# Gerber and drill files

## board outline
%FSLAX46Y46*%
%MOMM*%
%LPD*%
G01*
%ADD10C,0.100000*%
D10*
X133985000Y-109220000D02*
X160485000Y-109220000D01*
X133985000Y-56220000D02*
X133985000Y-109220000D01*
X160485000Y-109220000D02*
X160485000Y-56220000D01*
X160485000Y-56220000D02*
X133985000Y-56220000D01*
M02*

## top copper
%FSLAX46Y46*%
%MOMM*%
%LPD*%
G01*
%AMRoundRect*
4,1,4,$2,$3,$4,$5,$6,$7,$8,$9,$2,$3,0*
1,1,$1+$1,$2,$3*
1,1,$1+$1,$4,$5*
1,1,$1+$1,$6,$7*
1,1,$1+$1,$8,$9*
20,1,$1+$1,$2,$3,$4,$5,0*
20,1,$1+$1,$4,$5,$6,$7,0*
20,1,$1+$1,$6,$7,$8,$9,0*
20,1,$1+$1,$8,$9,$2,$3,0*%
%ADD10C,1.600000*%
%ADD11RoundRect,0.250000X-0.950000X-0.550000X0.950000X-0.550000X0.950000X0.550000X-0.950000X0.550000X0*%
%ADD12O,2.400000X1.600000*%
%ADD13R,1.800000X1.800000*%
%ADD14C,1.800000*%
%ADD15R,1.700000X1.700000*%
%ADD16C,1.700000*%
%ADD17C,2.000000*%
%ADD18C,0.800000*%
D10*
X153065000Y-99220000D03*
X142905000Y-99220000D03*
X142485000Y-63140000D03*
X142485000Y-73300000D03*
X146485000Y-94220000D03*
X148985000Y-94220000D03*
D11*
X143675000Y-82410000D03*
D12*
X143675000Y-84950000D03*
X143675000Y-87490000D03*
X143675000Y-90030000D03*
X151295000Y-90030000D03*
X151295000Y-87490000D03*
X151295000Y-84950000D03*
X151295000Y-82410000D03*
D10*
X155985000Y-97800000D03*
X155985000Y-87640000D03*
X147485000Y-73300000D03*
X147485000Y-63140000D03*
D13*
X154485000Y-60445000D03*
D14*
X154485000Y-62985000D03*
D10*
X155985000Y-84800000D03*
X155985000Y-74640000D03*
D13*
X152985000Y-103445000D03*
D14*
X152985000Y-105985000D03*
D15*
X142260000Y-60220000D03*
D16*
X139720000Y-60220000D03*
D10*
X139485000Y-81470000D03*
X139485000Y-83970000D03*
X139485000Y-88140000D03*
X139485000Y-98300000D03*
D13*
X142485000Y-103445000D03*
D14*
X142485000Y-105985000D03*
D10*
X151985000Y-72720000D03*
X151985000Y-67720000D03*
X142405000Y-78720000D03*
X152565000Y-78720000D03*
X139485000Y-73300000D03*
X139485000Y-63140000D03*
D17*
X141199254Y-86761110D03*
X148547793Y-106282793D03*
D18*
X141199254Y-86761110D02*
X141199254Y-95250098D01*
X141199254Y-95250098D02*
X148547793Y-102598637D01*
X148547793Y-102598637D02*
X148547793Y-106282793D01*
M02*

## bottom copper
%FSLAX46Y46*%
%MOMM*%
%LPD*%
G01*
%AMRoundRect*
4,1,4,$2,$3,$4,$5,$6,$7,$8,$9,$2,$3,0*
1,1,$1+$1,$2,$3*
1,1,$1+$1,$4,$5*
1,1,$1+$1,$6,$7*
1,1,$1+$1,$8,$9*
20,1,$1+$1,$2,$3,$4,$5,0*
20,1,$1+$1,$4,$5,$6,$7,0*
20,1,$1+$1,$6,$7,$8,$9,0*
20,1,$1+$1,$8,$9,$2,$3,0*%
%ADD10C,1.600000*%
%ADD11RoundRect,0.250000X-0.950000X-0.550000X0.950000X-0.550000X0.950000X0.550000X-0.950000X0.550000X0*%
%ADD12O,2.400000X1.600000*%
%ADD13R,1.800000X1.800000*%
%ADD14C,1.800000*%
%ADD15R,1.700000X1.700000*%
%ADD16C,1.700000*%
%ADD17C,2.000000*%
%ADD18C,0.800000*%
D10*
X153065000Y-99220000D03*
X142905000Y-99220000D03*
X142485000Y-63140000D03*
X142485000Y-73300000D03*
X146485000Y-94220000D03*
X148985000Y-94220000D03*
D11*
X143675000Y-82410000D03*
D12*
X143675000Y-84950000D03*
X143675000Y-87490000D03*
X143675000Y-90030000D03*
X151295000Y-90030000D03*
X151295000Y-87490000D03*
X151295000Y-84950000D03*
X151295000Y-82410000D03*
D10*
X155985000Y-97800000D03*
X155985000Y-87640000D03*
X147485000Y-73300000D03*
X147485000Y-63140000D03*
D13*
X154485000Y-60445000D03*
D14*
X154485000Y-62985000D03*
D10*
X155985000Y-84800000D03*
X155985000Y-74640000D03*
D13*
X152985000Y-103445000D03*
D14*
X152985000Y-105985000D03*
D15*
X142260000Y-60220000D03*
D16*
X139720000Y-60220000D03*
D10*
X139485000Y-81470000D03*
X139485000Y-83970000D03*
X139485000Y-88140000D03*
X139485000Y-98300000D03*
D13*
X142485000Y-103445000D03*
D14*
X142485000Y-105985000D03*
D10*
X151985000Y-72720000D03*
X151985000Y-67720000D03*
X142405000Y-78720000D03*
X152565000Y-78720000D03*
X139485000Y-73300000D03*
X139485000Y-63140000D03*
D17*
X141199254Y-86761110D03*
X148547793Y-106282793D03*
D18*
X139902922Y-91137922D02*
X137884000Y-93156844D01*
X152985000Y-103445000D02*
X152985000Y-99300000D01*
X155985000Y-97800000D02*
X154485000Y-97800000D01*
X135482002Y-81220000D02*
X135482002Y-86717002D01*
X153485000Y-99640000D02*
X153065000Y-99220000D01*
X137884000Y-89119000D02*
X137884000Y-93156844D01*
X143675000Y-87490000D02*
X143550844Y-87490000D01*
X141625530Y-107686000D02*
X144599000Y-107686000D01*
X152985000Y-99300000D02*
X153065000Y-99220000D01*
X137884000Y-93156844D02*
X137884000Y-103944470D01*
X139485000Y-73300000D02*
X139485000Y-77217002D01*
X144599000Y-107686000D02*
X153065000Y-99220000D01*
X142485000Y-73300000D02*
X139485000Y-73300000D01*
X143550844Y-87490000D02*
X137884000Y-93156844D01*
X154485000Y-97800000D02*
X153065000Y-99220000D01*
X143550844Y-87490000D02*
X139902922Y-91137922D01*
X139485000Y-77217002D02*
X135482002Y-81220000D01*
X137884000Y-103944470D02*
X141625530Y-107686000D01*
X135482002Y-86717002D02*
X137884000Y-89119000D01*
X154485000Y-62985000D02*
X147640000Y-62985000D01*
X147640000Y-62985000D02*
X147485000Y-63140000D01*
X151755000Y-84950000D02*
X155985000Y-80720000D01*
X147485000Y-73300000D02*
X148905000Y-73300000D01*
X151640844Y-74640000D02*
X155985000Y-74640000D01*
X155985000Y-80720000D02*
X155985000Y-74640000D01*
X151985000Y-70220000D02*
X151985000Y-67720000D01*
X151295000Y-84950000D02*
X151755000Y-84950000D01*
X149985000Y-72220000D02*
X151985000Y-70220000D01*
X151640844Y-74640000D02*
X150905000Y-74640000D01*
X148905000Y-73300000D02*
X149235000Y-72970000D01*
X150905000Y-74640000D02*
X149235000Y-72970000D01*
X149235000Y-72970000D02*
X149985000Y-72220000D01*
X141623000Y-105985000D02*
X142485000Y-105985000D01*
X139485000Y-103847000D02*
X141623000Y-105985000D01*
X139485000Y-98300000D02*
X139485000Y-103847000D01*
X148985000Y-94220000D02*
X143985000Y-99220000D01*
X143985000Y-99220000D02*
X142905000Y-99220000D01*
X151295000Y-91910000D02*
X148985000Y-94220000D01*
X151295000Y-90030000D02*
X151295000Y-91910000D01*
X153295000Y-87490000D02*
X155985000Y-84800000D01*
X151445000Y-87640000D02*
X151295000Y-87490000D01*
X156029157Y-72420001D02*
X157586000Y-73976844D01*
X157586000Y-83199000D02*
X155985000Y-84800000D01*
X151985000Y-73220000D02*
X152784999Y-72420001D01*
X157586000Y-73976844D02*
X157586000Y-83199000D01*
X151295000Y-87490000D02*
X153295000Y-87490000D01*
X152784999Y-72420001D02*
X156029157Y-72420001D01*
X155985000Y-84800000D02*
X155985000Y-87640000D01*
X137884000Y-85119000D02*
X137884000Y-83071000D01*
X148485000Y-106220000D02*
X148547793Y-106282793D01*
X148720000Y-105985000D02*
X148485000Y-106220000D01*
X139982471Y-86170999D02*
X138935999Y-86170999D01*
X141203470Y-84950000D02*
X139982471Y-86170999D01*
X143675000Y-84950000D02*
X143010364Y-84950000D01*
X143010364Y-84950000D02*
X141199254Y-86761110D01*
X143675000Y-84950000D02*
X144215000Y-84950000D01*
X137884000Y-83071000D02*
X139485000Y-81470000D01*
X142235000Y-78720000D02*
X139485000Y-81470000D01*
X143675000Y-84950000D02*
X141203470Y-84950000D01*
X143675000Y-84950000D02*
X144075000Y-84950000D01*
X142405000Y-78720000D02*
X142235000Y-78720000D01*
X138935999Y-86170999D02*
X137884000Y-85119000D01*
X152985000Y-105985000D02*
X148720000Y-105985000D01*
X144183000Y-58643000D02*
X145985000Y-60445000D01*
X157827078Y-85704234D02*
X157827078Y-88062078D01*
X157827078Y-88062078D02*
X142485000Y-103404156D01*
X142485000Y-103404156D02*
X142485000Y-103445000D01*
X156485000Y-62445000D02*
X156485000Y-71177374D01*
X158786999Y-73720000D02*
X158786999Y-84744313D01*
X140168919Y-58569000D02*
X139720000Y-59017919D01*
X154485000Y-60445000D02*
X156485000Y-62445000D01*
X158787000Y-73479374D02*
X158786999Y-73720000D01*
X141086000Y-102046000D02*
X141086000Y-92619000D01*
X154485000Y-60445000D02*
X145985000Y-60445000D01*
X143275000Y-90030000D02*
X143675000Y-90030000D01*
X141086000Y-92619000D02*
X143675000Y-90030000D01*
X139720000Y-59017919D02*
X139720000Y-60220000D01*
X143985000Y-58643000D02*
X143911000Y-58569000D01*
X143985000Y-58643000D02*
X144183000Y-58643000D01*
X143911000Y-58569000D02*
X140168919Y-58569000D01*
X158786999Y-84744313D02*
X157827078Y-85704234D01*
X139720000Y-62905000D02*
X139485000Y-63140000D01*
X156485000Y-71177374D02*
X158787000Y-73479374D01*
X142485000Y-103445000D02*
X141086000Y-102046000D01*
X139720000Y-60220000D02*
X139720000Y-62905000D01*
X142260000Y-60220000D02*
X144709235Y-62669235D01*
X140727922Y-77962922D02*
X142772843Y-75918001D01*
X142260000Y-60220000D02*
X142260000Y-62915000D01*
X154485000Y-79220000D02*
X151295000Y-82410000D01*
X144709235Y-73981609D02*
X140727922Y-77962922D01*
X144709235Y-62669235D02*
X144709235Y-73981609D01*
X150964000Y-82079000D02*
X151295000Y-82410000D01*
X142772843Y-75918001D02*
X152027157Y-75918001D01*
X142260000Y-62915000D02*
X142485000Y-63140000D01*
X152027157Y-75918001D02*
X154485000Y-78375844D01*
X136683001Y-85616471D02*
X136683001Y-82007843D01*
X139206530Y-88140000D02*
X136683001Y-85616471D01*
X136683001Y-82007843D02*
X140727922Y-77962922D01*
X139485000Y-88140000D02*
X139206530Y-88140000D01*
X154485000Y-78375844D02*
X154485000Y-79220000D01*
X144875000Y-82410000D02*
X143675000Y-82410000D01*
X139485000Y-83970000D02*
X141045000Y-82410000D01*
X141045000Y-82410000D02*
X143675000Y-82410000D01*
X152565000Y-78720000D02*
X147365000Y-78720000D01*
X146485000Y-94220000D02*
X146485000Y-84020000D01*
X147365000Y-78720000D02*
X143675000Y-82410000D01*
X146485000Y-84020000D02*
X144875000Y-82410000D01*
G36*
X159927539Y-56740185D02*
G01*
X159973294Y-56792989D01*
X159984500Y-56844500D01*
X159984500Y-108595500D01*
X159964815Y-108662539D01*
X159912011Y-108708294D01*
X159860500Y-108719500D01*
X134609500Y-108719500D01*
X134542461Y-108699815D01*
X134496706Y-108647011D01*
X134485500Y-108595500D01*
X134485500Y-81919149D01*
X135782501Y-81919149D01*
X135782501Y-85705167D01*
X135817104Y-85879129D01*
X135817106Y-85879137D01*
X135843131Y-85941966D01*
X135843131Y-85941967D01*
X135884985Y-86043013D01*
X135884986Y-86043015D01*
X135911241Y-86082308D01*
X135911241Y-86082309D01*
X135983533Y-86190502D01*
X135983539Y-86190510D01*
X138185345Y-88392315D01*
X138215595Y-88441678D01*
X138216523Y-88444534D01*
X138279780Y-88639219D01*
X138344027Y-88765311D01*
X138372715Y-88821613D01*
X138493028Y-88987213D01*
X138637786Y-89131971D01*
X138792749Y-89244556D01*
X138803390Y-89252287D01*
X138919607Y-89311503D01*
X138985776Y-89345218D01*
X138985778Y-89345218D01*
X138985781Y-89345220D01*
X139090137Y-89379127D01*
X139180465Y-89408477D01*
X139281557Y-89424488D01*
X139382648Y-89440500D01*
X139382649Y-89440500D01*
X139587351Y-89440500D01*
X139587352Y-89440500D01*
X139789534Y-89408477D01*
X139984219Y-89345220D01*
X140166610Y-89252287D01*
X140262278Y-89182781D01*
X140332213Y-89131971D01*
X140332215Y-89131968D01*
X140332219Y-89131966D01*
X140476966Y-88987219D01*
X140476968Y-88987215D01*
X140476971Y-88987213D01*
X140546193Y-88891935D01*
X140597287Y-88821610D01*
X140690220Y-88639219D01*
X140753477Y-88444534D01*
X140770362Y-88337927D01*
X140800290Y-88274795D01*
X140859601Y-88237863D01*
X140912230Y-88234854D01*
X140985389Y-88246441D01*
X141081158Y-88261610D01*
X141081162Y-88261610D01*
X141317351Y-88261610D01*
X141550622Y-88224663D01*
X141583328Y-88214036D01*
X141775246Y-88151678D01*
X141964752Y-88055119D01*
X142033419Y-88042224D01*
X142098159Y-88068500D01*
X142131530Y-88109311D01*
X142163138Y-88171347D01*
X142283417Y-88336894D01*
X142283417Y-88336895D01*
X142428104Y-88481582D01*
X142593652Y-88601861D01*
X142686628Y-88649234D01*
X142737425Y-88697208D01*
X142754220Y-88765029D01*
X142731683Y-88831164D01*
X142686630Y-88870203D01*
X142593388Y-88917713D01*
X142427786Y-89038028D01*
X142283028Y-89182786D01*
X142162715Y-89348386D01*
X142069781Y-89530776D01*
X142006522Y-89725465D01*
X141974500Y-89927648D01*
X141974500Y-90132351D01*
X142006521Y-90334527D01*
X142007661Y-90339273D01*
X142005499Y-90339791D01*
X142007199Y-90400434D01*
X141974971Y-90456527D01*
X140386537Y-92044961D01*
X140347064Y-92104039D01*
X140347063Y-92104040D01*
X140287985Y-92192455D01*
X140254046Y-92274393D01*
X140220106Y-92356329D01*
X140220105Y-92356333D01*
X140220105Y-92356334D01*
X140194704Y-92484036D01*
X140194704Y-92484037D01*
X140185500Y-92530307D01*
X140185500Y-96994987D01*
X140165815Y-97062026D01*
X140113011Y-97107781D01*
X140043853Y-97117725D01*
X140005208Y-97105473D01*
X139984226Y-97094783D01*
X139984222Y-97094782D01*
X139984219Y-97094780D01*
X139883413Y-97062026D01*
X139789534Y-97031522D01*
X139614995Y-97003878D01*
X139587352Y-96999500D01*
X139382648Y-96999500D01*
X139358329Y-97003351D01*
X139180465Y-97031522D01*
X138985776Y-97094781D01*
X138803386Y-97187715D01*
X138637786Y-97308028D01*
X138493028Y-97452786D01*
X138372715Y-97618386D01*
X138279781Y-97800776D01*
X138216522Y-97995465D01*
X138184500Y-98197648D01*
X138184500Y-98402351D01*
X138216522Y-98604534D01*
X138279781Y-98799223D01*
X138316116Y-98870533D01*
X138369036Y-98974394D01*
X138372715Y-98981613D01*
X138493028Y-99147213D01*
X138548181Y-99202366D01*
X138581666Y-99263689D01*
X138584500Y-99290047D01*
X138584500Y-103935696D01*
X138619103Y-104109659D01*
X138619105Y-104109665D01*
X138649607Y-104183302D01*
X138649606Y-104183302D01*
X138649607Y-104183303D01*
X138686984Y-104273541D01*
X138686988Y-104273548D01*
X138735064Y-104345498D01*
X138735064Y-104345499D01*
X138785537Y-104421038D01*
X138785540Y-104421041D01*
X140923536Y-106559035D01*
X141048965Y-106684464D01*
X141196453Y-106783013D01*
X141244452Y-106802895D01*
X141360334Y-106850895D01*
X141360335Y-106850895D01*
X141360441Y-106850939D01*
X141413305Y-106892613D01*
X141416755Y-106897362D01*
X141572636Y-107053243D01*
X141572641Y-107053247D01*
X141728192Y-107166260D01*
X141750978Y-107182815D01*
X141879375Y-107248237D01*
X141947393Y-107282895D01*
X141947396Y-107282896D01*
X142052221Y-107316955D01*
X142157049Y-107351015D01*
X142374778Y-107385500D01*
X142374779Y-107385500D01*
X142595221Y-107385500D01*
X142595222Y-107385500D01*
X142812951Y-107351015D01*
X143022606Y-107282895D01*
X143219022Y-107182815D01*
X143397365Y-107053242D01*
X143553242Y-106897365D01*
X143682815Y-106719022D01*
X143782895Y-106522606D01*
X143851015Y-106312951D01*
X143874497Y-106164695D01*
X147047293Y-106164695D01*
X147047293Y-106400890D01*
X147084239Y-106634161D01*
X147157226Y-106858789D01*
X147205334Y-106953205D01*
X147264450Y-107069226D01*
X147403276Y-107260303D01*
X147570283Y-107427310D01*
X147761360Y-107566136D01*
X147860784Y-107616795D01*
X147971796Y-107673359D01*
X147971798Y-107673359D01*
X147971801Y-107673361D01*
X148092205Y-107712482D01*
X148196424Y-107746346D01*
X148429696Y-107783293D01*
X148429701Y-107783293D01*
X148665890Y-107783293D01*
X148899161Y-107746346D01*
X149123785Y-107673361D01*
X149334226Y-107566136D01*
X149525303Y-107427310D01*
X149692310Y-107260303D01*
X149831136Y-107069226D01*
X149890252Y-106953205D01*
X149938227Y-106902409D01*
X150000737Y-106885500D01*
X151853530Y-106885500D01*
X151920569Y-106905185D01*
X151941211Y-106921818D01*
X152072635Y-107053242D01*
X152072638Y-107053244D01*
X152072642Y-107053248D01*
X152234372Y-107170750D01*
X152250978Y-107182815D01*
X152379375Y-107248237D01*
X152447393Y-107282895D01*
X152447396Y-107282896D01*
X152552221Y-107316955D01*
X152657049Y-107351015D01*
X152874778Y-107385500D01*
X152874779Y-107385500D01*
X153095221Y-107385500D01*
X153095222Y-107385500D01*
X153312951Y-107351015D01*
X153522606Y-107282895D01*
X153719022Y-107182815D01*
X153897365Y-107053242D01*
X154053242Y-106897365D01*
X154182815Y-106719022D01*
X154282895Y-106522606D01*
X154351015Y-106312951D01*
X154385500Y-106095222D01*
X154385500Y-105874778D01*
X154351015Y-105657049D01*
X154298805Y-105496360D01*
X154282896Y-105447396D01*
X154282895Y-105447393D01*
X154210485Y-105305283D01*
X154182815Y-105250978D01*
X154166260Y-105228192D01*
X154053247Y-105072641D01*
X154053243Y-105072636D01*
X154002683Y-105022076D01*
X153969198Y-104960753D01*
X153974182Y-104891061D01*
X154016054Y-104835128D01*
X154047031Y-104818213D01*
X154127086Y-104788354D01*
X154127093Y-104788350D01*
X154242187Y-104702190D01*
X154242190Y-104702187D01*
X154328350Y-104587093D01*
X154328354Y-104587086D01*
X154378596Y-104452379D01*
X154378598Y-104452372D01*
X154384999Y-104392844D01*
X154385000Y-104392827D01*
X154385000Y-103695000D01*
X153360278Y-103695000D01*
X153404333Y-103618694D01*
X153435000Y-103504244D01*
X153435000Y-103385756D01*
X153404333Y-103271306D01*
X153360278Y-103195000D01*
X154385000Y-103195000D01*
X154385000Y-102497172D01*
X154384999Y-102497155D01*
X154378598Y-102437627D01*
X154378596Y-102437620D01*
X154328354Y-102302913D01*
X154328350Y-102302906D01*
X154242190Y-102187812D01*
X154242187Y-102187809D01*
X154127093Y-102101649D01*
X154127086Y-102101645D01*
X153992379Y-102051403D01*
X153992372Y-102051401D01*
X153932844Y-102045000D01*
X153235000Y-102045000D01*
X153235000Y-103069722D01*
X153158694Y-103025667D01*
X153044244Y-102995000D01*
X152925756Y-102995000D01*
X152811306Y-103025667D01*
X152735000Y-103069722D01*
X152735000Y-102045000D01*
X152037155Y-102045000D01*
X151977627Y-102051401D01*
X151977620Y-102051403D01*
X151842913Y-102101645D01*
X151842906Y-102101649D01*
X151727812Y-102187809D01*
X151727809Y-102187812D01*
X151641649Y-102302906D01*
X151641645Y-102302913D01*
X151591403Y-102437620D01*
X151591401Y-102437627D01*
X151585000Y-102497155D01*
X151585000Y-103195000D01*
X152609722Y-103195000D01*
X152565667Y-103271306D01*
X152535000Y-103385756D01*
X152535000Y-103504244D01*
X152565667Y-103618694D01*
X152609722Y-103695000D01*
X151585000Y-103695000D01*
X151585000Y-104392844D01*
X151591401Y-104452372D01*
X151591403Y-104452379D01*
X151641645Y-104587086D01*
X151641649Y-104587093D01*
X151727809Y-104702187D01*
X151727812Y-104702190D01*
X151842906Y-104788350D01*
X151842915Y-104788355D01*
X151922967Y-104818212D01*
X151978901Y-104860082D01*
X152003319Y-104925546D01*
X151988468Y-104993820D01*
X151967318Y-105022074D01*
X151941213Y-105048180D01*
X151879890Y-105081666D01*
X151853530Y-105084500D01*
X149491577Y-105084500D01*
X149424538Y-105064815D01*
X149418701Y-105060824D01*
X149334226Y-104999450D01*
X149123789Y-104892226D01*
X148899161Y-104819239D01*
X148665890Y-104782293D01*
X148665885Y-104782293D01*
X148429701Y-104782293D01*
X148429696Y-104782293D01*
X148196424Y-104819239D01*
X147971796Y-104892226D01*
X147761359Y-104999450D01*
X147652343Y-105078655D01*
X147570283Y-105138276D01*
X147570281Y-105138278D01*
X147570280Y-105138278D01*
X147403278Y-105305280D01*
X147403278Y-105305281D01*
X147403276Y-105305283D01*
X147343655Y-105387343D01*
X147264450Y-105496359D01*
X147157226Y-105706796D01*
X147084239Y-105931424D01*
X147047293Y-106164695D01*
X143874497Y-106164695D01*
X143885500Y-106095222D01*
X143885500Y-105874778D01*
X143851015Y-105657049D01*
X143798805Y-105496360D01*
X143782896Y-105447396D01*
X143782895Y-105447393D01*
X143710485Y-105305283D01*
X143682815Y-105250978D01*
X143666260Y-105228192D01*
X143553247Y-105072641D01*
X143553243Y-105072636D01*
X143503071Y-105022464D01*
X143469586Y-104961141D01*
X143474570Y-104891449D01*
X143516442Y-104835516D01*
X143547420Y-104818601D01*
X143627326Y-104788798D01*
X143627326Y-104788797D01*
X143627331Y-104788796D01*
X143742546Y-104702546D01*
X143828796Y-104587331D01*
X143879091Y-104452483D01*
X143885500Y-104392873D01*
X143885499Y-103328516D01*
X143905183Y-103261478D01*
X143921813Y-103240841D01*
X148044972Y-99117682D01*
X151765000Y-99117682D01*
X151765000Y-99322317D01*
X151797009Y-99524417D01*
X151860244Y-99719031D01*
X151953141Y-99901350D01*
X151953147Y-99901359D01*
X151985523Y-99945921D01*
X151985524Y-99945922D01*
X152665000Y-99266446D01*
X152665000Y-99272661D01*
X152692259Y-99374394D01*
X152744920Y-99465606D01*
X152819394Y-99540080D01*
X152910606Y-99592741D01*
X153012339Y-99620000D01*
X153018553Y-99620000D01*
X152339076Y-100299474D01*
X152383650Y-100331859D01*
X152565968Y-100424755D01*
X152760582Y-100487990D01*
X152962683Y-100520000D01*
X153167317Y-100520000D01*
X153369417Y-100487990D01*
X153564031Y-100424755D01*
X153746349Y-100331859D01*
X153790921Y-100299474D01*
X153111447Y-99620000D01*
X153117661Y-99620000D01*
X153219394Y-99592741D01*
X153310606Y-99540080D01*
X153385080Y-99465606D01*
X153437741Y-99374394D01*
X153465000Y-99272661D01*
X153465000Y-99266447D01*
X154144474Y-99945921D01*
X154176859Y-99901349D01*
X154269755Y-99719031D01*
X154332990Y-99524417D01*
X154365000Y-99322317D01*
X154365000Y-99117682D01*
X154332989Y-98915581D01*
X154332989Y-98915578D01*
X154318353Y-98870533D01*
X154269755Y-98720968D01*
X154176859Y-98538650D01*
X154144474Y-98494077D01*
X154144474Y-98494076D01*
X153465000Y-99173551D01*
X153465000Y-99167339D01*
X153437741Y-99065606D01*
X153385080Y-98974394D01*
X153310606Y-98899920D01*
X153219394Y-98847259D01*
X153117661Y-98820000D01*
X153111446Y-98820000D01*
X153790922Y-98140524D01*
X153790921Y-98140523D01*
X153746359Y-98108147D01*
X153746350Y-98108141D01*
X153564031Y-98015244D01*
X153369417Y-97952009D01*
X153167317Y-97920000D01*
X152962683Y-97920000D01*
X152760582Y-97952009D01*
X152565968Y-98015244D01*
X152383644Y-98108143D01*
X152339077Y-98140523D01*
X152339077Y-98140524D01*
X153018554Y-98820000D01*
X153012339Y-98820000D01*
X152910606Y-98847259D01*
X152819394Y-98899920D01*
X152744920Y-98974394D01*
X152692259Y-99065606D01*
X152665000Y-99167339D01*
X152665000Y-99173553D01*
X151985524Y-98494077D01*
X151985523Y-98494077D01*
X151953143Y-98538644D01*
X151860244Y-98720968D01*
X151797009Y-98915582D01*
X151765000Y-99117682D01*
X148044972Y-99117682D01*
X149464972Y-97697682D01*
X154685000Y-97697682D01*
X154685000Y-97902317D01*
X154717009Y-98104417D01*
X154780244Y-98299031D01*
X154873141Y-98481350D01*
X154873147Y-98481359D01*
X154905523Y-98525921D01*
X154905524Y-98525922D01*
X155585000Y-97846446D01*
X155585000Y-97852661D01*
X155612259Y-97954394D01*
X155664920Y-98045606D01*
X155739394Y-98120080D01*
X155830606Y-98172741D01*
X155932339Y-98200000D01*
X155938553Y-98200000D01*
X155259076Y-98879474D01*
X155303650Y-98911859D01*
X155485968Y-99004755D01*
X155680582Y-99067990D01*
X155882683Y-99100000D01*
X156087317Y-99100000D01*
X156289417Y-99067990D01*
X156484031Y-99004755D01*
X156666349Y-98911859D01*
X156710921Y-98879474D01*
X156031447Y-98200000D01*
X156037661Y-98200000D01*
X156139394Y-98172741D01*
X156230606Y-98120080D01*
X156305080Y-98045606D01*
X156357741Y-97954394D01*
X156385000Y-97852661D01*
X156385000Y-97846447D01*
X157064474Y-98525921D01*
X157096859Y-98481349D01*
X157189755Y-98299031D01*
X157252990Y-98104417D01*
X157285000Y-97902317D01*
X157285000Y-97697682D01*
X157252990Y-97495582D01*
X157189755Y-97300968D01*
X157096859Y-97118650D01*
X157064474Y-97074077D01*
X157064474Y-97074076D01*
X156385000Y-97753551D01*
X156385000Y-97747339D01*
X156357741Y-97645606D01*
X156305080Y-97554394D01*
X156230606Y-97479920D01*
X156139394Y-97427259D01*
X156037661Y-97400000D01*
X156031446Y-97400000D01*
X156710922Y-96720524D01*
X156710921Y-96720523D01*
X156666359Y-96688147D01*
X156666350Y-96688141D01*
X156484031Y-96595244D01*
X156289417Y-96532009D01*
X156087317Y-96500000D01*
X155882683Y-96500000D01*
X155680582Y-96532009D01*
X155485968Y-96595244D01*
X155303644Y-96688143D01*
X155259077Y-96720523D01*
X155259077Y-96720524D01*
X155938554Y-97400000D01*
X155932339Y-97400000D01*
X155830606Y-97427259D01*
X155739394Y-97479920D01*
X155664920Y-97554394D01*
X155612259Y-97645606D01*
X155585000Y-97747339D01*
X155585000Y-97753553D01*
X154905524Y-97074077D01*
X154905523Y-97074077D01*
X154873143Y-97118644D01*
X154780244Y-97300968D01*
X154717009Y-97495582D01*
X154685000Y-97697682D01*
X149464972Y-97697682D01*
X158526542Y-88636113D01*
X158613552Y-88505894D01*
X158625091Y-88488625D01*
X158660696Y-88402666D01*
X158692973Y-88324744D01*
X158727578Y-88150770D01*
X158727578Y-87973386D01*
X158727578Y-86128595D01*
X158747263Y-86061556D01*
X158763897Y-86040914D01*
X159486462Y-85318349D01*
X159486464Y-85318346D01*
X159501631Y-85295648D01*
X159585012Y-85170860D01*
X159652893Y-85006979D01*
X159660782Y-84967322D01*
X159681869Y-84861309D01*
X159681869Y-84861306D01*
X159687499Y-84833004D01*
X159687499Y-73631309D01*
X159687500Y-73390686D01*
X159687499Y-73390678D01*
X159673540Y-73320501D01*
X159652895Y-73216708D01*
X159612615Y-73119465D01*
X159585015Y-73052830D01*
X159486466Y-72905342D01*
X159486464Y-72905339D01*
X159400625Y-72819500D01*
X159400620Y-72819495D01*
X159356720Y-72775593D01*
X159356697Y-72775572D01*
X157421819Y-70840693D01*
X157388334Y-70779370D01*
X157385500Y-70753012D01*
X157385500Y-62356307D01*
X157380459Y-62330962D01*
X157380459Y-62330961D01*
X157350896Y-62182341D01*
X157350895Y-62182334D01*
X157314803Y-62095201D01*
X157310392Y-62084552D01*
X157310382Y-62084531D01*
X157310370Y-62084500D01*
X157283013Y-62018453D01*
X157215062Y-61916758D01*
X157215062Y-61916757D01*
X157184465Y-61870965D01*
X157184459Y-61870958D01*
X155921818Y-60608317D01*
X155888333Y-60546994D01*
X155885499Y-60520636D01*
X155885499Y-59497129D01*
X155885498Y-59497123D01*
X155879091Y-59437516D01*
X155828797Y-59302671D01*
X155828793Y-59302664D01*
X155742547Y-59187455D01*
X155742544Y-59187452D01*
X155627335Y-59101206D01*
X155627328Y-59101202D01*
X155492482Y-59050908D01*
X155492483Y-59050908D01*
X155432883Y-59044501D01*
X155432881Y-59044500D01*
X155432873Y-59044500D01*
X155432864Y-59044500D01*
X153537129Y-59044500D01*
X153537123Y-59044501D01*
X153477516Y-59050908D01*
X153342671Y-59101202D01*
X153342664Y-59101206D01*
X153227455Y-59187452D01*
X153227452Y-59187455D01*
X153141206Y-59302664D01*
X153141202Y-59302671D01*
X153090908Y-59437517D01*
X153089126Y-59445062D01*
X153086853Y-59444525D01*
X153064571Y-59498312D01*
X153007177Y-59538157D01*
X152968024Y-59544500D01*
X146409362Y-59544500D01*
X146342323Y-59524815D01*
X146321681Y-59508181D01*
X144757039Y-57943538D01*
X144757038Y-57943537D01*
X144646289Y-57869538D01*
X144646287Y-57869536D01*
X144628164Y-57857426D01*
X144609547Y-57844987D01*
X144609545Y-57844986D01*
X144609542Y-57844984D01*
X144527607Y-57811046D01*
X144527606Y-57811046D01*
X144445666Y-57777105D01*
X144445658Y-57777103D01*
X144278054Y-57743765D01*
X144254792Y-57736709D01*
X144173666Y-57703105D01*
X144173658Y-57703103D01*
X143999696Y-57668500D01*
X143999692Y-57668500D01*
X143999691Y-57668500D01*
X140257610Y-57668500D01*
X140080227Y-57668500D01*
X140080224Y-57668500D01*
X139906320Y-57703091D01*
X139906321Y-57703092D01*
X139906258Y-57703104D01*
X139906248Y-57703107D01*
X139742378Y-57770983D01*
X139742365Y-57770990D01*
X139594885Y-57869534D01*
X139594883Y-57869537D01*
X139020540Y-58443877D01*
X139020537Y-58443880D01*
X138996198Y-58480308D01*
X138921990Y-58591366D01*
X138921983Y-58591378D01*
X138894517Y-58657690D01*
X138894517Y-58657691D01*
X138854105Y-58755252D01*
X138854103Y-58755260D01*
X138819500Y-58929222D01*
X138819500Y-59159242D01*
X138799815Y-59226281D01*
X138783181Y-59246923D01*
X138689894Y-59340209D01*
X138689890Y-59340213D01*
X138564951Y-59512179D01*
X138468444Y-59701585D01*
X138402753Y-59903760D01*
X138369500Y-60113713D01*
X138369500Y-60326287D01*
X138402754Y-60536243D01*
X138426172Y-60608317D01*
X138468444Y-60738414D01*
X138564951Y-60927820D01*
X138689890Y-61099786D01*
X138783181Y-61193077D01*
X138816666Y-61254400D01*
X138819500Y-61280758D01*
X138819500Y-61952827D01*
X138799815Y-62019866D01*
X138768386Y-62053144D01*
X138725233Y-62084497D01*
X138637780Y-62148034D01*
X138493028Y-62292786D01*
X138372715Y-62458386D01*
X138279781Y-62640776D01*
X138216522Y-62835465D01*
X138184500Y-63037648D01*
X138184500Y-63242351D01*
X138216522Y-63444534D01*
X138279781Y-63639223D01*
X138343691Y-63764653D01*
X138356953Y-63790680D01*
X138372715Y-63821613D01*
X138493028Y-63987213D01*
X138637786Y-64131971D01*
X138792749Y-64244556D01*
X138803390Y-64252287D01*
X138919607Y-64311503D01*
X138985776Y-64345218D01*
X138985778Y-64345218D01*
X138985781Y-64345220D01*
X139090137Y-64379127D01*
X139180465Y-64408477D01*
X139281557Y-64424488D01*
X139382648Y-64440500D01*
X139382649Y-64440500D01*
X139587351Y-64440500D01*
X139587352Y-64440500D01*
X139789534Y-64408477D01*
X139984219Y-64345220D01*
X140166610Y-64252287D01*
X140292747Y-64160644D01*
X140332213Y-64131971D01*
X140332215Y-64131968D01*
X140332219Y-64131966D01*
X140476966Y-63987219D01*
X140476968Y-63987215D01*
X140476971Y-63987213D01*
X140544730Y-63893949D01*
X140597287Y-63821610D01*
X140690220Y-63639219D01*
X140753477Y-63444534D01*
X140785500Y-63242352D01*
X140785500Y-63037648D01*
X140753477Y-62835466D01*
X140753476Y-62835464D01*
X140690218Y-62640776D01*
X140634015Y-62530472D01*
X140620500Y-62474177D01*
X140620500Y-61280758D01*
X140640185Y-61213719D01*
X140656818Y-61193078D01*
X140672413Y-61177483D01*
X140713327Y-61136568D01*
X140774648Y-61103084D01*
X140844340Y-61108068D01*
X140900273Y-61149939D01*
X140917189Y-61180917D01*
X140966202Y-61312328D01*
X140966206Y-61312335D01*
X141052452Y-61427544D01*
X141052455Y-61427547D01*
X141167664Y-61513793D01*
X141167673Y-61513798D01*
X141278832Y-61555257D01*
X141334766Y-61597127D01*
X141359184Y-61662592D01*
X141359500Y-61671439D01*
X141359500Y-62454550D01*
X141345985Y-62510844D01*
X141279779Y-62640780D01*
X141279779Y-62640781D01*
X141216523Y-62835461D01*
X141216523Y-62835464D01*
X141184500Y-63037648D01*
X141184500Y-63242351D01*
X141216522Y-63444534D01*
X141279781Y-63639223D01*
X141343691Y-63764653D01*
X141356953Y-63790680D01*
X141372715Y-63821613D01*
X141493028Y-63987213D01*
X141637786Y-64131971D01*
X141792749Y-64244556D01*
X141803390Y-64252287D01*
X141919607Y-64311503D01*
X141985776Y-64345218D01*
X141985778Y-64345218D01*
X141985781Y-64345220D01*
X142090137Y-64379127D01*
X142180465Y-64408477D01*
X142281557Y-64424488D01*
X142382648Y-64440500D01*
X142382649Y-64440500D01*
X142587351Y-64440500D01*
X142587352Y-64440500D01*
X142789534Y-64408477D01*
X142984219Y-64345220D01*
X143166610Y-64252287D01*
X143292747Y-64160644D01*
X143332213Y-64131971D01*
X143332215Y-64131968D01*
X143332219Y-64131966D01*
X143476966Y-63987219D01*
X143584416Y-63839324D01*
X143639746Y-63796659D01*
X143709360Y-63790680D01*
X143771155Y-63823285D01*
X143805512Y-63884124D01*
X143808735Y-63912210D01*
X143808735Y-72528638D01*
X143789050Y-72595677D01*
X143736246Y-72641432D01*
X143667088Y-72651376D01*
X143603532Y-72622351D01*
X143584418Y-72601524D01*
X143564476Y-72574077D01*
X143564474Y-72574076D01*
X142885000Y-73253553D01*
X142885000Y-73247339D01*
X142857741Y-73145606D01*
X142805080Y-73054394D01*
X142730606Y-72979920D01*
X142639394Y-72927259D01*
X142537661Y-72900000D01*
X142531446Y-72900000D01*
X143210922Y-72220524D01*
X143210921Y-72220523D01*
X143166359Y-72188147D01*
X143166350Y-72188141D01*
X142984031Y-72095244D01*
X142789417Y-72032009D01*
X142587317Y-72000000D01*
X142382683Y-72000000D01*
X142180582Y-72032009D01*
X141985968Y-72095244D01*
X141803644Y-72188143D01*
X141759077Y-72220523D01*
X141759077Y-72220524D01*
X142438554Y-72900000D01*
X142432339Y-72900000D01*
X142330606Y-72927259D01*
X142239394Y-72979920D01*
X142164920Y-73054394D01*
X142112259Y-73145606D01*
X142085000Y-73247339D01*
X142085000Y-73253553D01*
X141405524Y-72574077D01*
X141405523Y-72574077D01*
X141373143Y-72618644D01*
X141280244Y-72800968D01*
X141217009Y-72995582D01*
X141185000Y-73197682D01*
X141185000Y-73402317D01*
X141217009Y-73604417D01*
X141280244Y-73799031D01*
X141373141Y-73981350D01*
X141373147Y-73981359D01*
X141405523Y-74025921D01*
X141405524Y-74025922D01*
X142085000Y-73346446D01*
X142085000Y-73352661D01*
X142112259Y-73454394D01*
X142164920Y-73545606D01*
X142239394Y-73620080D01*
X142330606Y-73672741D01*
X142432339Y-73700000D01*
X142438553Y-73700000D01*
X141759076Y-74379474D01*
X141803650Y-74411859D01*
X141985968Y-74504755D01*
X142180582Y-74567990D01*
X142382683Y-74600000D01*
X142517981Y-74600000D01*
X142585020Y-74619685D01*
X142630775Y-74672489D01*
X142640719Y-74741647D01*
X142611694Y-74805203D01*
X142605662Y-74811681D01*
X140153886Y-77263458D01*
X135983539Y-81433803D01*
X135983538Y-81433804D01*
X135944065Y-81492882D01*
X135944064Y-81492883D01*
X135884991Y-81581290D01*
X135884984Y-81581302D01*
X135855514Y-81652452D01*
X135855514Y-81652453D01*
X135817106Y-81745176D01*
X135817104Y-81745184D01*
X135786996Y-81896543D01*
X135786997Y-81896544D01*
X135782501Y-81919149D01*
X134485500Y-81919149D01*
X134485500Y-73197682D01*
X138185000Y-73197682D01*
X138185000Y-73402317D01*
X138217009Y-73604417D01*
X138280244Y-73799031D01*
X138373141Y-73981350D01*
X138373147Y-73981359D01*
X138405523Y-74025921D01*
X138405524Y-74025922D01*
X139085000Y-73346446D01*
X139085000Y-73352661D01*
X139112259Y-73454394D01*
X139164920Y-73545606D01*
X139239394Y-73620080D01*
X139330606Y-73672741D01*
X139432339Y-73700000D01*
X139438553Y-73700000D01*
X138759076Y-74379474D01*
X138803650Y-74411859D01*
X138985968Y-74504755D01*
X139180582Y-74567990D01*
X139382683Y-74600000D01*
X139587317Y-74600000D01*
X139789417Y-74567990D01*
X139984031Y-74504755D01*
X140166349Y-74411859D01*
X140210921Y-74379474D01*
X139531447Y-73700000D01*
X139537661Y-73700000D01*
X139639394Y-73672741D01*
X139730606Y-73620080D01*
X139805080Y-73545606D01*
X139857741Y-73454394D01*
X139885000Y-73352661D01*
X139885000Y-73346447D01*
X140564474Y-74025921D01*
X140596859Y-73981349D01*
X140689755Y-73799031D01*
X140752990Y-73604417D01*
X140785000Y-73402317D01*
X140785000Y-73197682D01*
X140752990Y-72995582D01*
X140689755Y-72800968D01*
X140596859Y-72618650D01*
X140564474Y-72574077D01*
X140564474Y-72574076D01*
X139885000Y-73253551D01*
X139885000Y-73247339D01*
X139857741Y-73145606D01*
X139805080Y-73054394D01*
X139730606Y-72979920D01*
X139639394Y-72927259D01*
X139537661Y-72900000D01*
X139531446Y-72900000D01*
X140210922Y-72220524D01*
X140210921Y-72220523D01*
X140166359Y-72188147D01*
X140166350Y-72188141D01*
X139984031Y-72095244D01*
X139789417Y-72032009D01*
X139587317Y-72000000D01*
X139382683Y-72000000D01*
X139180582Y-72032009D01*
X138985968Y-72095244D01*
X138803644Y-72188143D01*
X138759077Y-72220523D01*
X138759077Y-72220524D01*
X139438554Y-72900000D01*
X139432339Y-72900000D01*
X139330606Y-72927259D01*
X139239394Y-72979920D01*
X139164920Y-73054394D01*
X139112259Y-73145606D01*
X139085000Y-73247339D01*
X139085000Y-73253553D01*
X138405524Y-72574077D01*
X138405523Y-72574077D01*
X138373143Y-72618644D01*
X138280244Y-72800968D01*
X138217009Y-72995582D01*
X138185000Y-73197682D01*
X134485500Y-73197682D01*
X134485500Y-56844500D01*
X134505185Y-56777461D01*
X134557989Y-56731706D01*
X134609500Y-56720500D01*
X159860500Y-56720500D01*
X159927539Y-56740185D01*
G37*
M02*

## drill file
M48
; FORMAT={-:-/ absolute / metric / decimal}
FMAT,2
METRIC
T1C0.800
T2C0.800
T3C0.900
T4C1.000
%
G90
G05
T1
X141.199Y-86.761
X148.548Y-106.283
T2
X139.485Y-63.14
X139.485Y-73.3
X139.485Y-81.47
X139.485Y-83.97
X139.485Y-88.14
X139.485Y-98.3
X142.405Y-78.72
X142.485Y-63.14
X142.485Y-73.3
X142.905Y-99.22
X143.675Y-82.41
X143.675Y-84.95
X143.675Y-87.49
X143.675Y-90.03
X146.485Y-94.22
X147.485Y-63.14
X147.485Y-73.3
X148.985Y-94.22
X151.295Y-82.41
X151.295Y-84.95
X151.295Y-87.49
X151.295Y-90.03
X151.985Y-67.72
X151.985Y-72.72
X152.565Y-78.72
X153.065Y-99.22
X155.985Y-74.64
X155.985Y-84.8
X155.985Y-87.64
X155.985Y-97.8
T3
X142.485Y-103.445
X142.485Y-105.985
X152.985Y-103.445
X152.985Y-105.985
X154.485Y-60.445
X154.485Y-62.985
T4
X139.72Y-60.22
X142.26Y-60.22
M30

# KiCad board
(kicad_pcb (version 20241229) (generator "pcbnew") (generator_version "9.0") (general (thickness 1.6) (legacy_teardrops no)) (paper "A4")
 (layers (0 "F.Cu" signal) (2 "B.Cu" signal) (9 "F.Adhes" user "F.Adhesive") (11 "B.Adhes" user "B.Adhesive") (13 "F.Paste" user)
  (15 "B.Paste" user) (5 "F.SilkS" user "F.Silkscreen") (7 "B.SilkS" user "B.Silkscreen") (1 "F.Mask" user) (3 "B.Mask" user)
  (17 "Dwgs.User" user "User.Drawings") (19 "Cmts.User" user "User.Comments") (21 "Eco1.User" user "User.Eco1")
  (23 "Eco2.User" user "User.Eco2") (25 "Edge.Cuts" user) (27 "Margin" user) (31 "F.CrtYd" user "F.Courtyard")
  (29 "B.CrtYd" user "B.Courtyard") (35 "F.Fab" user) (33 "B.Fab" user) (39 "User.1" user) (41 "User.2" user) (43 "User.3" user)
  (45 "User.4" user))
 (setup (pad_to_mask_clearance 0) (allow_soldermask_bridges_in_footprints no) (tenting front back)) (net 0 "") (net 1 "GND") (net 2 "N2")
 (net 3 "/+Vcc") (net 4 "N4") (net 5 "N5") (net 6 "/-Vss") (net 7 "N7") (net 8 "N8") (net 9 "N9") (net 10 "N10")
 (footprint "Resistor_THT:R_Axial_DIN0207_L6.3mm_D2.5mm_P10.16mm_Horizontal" (layer "F.Cu") (at 153.065 99.22 180)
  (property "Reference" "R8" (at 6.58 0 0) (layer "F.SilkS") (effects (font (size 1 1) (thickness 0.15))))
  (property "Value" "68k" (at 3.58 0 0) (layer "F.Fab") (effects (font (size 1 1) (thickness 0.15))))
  (pad "1" thru_hole circle (at 0 0 180) (size 1.6 1.6) (drill 0.8) (layers "*.Cu" "*.Mask") (remove_unused_layers no) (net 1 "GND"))
  (pad "2" thru_hole circle (at 10.16 0 180) (size 1.6 1.6) (drill 0.8) (layers "*.Cu" "*.Mask") (remove_unused_layers no) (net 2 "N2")))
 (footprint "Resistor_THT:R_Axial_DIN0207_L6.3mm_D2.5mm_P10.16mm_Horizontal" (layer "F.Cu") (at 142.485 63.14 -90)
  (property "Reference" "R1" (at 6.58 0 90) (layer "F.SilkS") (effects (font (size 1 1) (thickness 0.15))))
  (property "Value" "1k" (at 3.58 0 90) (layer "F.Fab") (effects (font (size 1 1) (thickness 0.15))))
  (pad "1" thru_hole circle (at 0 0 270) (size 1.6 1.6) (drill 0.8) (layers "*.Cu" "*.Mask") (remove_unused_layers no) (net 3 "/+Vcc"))
  (pad "2" thru_hole circle (at 10.16 0 270) (size 1.6 1.6) (drill 0.8) (layers "*.Cu" "*.Mask") (remove_unused_layers no) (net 1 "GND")))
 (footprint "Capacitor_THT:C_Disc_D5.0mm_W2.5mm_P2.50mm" (layer "F.Cu") (at 146.485 94.22)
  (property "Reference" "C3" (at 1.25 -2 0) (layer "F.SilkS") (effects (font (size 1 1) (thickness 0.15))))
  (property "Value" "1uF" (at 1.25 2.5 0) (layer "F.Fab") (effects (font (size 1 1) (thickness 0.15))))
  (pad "1" thru_hole circle (at 0 0) (size 1.6 1.6) (drill 0.8) (layers "*.Cu" "*.Mask") (remove_unused_layers no) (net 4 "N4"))
  (pad "2" thru_hole circle (at 2.5 0) (size 1.6 1.6) (drill 0.8) (layers "*.Cu" "*.Mask") (remove_unused_layers no) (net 2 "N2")))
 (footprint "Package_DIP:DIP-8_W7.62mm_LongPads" (layer "F.Cu") (at 143.675 82.41)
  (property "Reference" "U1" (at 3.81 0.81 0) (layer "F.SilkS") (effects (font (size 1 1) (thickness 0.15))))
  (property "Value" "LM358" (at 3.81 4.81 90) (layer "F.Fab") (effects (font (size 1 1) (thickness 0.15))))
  (pad "1" thru_hole roundrect (at 0 0) (size 2.4 1.6) (drill 0.8) (layers "*.Cu" "*.Mask") (remove_unused_layers no)
   (roundrect_rratio 0.15625) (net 4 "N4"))
  (pad "2" thru_hole oval (at 0 2.54) (size 2.4 1.6) (drill 0.8) (layers "*.Cu" "*.Mask") (remove_unused_layers no) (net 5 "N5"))
  (pad "3" thru_hole oval (at 0 5.08) (size 2.4 1.6) (drill 0.8) (layers "*.Cu" "*.Mask") (remove_unused_layers no) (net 1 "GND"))
  (pad "4" thru_hole oval (at 0 7.62) (size 2.4 1.6) (drill 0.8) (layers "*.Cu" "*.Mask") (remove_unused_layers no) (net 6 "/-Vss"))
  (pad "5" thru_hole oval (at 7.62 7.62) (size 2.4 1.6) (drill 0.8) (layers "*.Cu" "*.Mask") (remove_unused_layers no) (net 2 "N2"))
  (pad "6" thru_hole oval (at 7.62 5.08) (size 2.4 1.6) (drill 0.8) (layers "*.Cu" "*.Mask") (remove_unused_layers no) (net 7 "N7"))
  (pad "7" thru_hole oval (at 7.62 2.54) (size 2.4 1.6) (drill 0.8) (layers "*.Cu" "*.Mask") (remove_unused_layers no) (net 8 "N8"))
  (pad "8" thru_hole oval (at 7.62 0) (size 2.4 1.6) (drill 0.8) (layers "*.Cu" "*.Mask") (remove_unused_layers no) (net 3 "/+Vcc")))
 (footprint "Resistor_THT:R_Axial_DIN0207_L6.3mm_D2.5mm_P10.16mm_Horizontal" (layer "F.Cu") (at 155.985 97.8 90)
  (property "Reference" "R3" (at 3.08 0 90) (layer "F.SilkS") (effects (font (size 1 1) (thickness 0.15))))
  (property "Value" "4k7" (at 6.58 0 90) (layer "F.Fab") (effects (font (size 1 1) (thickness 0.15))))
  (pad "1" thru_hole circle (at 0 0 90) (size 1.6 1.6) (drill 0.8) (layers "*.Cu" "*.Mask") (remove_unused_layers no) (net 1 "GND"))
  (pad "2" thru_hole circle (at 10.16 0 90) (size 1.6 1.6) (drill 0.8) (layers "*.Cu" "*.Mask") (remove_unused_layers no) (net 7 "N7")))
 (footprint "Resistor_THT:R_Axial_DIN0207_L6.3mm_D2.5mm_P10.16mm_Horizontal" (layer "F.Cu") (at 147.485 73.3 90)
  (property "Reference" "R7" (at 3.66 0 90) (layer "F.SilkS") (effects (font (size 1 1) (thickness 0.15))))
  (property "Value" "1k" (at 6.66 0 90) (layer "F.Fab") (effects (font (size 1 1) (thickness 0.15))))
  (pad "1" thru_hole circle (at 0 0 90) (size 1.6 1.6) (drill 0.8) (layers "*.Cu" "*.Mask") (remove_unused_layers no) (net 8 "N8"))
  (pad "2" thru_hole circle (at 10.16 0 90) (size 1.6 1.6) (drill 0.8) (layers "*.Cu" "*.Mask") (remove_unused_layers no) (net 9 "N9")))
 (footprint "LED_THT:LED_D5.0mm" (layer "F.Cu") (at 154.485 60.445 -90)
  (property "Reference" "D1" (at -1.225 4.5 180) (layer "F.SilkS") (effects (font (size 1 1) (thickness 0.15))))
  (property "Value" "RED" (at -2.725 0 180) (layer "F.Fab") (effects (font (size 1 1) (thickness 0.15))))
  (pad "1" thru_hole rect (at 0 0 270) (size 1.8 1.8) (drill 0.9) (layers "*.Cu" "*.Mask") (remove_unused_layers no) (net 6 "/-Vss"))
  (pad "2" thru_hole circle (at 2.54 0 270) (size 1.8 1.8) (drill 0.9) (layers "*.Cu" "*.Mask") (remove_unused_layers no) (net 9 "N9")))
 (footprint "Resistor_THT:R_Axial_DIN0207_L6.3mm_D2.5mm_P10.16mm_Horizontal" (layer "F.Cu") (at 155.985 84.8 90)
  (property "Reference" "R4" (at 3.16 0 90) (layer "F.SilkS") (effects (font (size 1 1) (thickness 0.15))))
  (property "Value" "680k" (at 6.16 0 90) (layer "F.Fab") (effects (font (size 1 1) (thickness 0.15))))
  (pad "1" thru_hole circle (at 0 0 90) (size 1.6 1.6) (drill 0.8) (layers "*.Cu" "*.Mask") (remove_unused_layers no) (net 7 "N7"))
  (pad "2" thru_hole circle (at 10.16 0 90) (size 1.6 1.6) (drill 0.8) (layers "*.Cu" "*.Mask") (remove_unused_layers no) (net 8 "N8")))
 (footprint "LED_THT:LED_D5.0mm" (layer "F.Cu") (at 152.985 103.445 -90)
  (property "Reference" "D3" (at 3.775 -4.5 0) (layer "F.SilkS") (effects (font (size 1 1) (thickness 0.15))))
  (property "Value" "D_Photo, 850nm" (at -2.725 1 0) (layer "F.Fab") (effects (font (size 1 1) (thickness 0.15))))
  (pad "1" thru_hole rect (at 0 0 270) (size 1.8 1.8) (drill 0.9) (layers "*.Cu" "*.Mask") (remove_unused_layers no) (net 1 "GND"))
  (pad "2" thru_hole circle (at 2.54 0 270) (size 1.8 1.8) (drill 0.9) (layers "*.Cu" "*.Mask") (remove_unused_layers no) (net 5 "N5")))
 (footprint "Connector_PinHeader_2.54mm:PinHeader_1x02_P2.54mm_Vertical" (layer "F.Cu") (at 142.26 60.22 -90)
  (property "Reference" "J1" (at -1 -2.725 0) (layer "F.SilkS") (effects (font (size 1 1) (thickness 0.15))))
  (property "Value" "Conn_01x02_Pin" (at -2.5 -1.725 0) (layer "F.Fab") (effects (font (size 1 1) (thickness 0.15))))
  (pad "1" thru_hole rect (at 0 0 270) (size 1.7 1.7) (drill 1) (layers "*.Cu" "*.Mask") (remove_unused_layers no) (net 3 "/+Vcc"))
  (pad "2" thru_hole circle (at 0 2.54 270) (size 1.7 1.7) (drill 1) (layers "*.Cu" "*.Mask") (remove_unused_layers no) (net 6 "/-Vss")))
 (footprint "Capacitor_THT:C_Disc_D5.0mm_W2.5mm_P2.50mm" (layer "F.Cu") (at 139.485 81.47 -90)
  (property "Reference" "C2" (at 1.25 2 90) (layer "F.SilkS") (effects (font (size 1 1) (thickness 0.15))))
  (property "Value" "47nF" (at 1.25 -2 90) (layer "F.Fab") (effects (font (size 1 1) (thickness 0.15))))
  (pad "1" thru_hole circle (at 0 0 270) (size 1.6 1.6) (drill 0.8) (layers "*.Cu" "*.Mask") (remove_unused_layers no) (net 5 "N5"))
  (pad "2" thru_hole circle (at 2.5 0 270) (size 1.6 1.6) (drill 0.8) (layers "*.Cu" "*.Mask") (remove_unused_layers no) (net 4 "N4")))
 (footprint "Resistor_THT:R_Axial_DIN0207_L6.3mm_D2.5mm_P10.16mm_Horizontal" (layer "F.Cu") (at 139.485 88.14 -90)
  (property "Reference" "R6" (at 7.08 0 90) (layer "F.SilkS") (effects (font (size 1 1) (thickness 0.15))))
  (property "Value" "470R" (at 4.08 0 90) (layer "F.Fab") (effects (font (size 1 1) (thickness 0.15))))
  (pad "1" thru_hole circle (at 0 0 270) (size 1.6 1.6) (drill 0.8) (layers "*.Cu" "*.Mask") (remove_unused_layers no) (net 3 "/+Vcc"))
  (pad "2" thru_hole circle (at 10.16 0 270) (size 1.6 1.6) (drill 0.8) (layers "*.Cu" "*.Mask") (remove_unused_layers no) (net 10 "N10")))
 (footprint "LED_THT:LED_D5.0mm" (layer "F.Cu") (at 142.485 103.445 -90)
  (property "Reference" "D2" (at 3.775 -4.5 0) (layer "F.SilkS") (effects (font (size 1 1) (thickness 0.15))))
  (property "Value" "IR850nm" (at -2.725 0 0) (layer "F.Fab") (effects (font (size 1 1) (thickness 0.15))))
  (pad "1" thru_hole rect (at 0 0 270) (size 1.8 1.8) (drill 0.9) (layers "*.Cu" "*.Mask") (remove_unused_layers no) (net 6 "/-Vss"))
  (pad "2" thru_hole circle (at 2.54 0 270) (size 1.8 1.8) (drill 0.9) (layers "*.Cu" "*.Mask") (remove_unused_layers no) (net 10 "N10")))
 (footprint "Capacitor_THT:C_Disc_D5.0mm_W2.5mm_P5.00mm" (layer "F.Cu") (at 151.985 72.72 90)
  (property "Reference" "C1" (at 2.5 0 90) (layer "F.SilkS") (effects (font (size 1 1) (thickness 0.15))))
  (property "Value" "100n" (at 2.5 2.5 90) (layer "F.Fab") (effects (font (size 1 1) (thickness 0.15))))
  (pad "1" thru_hole circle (at 0 0 90) (size 1.6 1.6) (drill 0.8) (layers "*.Cu" "*.Mask") (remove_unused_layers no) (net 7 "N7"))
  (pad "2" thru_hole circle (at 5 0 90) (size 1.6 1.6) (drill 0.8) (layers "*.Cu" "*.Mask") (remove_unused_layers no) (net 8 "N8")))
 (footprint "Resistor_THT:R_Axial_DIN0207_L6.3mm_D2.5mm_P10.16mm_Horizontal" (layer "F.Cu") (at 142.405 78.72)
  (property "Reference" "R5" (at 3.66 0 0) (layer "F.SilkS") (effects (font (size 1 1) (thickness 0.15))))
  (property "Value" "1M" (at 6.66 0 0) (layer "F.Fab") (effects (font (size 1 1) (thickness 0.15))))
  (pad "1" thru_hole circle (at 0 0) (size 1.6 1.6) (drill 0.8) (layers "*.Cu" "*.Mask") (remove_unused_layers no) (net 5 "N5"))
  (pad "2" thru_hole circle (at 10.16 0) (size 1.6 1.6) (drill 0.8) (layers "*.Cu" "*.Mask") (remove_unused_layers no) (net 4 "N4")))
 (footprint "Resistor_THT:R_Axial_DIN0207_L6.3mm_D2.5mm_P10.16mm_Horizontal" (layer "F.Cu") (at 139.485 73.3 90)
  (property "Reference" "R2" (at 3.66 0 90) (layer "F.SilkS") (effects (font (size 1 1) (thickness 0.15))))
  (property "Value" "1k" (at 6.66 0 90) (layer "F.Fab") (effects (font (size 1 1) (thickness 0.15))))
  (pad "1" thru_hole circle (at 0 0 90) (size 1.6 1.6) (drill 0.8) (layers "*.Cu" "*.Mask") (remove_unused_layers no) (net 1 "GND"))
  (pad "2" thru_hole circle (at 10.16 0 90) (size 1.6 1.6) (drill 0.8) (layers "*.Cu" "*.Mask") (remove_unused_layers no) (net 6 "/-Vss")))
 (gr_line (start 133.985 109.22) (end 160.485 109.22) (stroke (width 0.1) (type default)) (layer "Edge.Cuts"))
 (gr_line (start 133.985 56.22) (end 133.985 109.22) (stroke (width 0.1) (type default)) (layer "Edge.Cuts"))
 (gr_line (start 160.485 109.22) (end 160.485 56.22) (stroke (width 0.1) (type default)) (layer "Edge.Cuts"))
 (gr_line (start 160.485 56.22) (end 133.985 56.22) (stroke (width 0.1) (type default)) (layer "Edge.Cuts"))
 (segment (start 139.902922 91.137922) (end 137.884 93.156844) (width 0.8) (layer "B.Cu") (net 1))
 (segment (start 152.985 103.445) (end 152.985 99.3) (width 0.8) (layer "B.Cu") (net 1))
 (segment (start 155.985 97.8) (end 154.485 97.8) (width 0.8) (layer "B.Cu") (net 1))
 (segment (start 135.482002 81.22) (end 135.482002 86.717002) (width 0.8) (layer "B.Cu") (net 1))
 (segment (start 153.485 99.64) (end 153.065 99.22) (width 0.8) (layer "B.Cu") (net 1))
 (segment (start 137.884 89.119) (end 137.884 93.156844) (width 0.8) (layer "B.Cu") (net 1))
 (segment (start 143.675 87.49) (end 143.550844 87.49) (width 0.8) (layer "B.Cu") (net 1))
 (segment (start 141.62553 107.686) (end 144.599 107.686) (width 0.8) (layer "B.Cu") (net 1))
 (segment (start 152.985 99.3) (end 153.065 99.22) (width 0.8) (layer "B.Cu") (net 1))
 (segment (start 137.884 93.156844) (end 137.884 103.94447) (width 0.8) (layer "B.Cu") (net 1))
 (segment (start 139.485 73.3) (end 139.485 77.217002) (width 0.8) (layer "B.Cu") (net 1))
 (segment (start 144.599 107.686) (end 153.065 99.22) (width 0.8) (layer "B.Cu") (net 1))
 (segment (start 142.485 73.3) (end 139.485 73.3) (width 0.8) (layer "B.Cu") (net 1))
 (segment (start 143.550844 87.49) (end 137.884 93.156844) (width 0.8) (layer "B.Cu") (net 1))
 (segment (start 154.485 97.8) (end 153.065 99.22) (width 0.8) (layer "B.Cu") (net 1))
 (segment (start 143.550844 87.49) (end 139.902922 91.137922) (width 0.8) (layer "B.Cu") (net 1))
 (segment (start 139.485 77.217002) (end 135.482002 81.22) (width 0.8) (layer "B.Cu") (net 1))
 (segment (start 137.884 103.94447) (end 141.62553 107.686) (width 0.8) (layer "B.Cu") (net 1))
 (segment (start 135.482002 86.717002) (end 137.884 89.119) (width 0.8) (layer "B.Cu") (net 1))
 (segment (start 154.485 62.985) (end 147.64 62.985) (width 0.8) (layer "B.Cu") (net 9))
 (segment (start 147.64 62.985) (end 147.485 63.14) (width 0.8) (layer "B.Cu") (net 9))
 (segment (start 151.755 84.95) (end 155.985 80.72) (width 0.8) (layer "B.Cu") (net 8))
 (segment (start 147.485 73.3) (end 148.905 73.3) (width 0.8) (layer "B.Cu") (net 8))
 (segment (start 151.640844 74.64) (end 155.985 74.64) (width 0.8) (layer "B.Cu") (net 8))
 (segment (start 155.985 80.72) (end 155.985 74.64) (width 0.8) (layer "B.Cu") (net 8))
 (segment (start 151.985 70.22) (end 151.985 67.72) (width 0.8) (layer "B.Cu") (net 8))
 (segment (start 151.295 84.95) (end 151.755 84.95) (width 0.8) (layer "B.Cu") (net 8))
 (segment (start 149.985 72.22) (end 151.985 70.22) (width 0.8) (layer "B.Cu") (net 8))
 (segment (start 151.640844 74.64) (end 150.905 74.64) (width 0.8) (layer "B.Cu") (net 8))
 (segment (start 148.905 73.3) (end 149.235 72.97) (width 0.8) (layer "B.Cu") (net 8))
 (segment (start 150.905 74.64) (end 149.235 72.97) (width 0.8) (layer "B.Cu") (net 8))
 (segment (start 149.235 72.97) (end 149.985 72.22) (width 0.8) (layer "B.Cu") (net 8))
 (segment (start 141.623 105.985) (end 142.485 105.985) (width 0.8) (layer "B.Cu") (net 10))
 (segment (start 139.485 103.847) (end 141.623 105.985) (width 0.8) (layer "B.Cu") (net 10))
 (segment (start 139.485 98.3) (end 139.485 103.847) (width 0.8) (layer "B.Cu") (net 10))
 (segment (start 148.985 94.22) (end 143.985 99.22) (width 0.8) (layer "B.Cu") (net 2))
 (segment (start 143.985 99.22) (end 142.905 99.22) (width 0.8) (layer "B.Cu") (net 2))
 (segment (start 151.295 91.91) (end 148.985 94.22) (width 0.8) (layer "B.Cu") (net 2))
 (segment (start 151.295 90.03) (end 151.295 91.91) (width 0.8) (layer "B.Cu") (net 2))
 (segment (start 153.295 87.49) (end 155.985 84.8) (width 0.8) (layer "B.Cu") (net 7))
 (segment (start 151.445 87.64) (end 151.295 87.49) (width 0.8) (layer "B.Cu") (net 7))
 (segment (start 156.029157 72.420001) (end 157.586 73.976844) (width 0.8) (layer "B.Cu") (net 7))
 (segment (start 157.586 83.199) (end 155.985 84.8) (width 0.8) (layer "B.Cu") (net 7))
 (segment (start 151.985 73.22) (end 152.784999 72.420001) (width 0.8) (layer "B.Cu") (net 7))
 (segment (start 157.586 73.976844) (end 157.586 83.199) (width 0.8) (layer "B.Cu") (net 7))
 (segment (start 151.295 87.49) (end 153.295 87.49) (width 0.8) (layer "B.Cu") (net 7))
 (segment (start 152.784999 72.420001) (end 156.029157 72.420001) (width 0.8) (layer "B.Cu") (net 7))
 (segment (start 155.985 84.8) (end 155.985 87.64) (width 0.8) (layer "B.Cu") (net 7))
 (segment (start 141.199254 86.76111) (end 141.199254 95.250098) (width 0.8) (layer "F.Cu") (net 5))
 (segment (start 141.199254 95.250098) (end 148.547793 102.598637) (width 0.8) (layer "F.Cu") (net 5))
 (segment (start 148.547793 102.598637) (end 148.547793 106.282793) (width 0.8) (layer "F.Cu") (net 5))
 (via (at 141.199254 86.76111) (size 2) (drill 0.8) (layers "F.Cu" "B.Cu") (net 5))
 (via (at 148.547793 106.282793) (size 2) (drill 0.8) (layers "F.Cu" "B.Cu") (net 5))
 (segment (start 137.884 85.119) (end 137.884 83.071) (width 0.8) (layer "B.Cu") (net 5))
 (segment (start 148.485 106.22) (end 148.547793 106.282793) (width 0.8) (layer "B.Cu") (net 5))
 (segment (start 148.72 105.985) (end 148.485 106.22) (width 0.8) (layer "B.Cu") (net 5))
 (segment (start 139.982471 86.170999) (end 138.935999 86.170999) (width 0.8) (layer "B.Cu") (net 5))
 (segment (start 141.20347 84.95) (end 139.982471 86.170999) (width 0.8) (layer "B.Cu") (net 5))
 (segment (start 143.675 84.95) (end 143.010364 84.95) (width 0.8) (layer "B.Cu") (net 5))
 (segment (start 143.010364 84.95) (end 141.199254 86.76111) (width 0.8) (layer "B.Cu") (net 5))
 (segment (start 143.675 84.95) (end 144.215 84.95) (width 0.8) (layer "B.Cu") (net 5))
 (segment (start 137.884 83.071) (end 139.485 81.47) (width 0.8) (layer "B.Cu") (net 5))
 (segment (start 142.235 78.72) (end 139.485 81.47) (width 0.8) (layer "B.Cu") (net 5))
 (segment (start 143.675 84.95) (end 141.20347 84.95) (width 0.8) (layer "B.Cu") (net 5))
 (segment (start 143.675 84.95) (end 144.075 84.95) (width 0.8) (layer "B.Cu") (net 5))
 (segment (start 142.405 78.72) (end 142.235 78.72) (width 0.8) (layer "B.Cu") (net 5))
 (segment (start 138.935999 86.170999) (end 137.884 85.119) (width 0.8) (layer "B.Cu") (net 5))
 (segment (start 152.985 105.985) (end 148.72 105.985) (width 0.8) (layer "B.Cu") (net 5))
 (segment (start 144.183 58.643) (end 145.985 60.445) (width 0.8) (layer "B.Cu") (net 6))
 (segment (start 157.827078 85.704234) (end 157.827078 88.062078) (width 0.8) (layer "B.Cu") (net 6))
 (segment (start 157.827078 88.062078) (end 142.485 103.404156) (width 0.8) (layer "B.Cu") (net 6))
 (segment (start 142.485 103.404156) (end 142.485 103.445) (width 0.8) (layer "B.Cu") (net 6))
 (segment (start 156.485 62.445) (end 156.485 71.177374) (width 0.8) (layer "B.Cu") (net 6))
 (segment (start 158.786999 73.72) (end 158.786999 84.744313) (width 0.8) (layer "B.Cu") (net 6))
 (segment (start 140.168919 58.569) (end 139.72 59.017919) (width 0.8) (layer "B.Cu") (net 6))
 (segment (start 154.485 60.445) (end 156.485 62.445) (width 0.8) (layer "B.Cu") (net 6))
 (segment (start 158.787 73.479374) (end 158.786999 73.72) (width 0.8) (layer "B.Cu") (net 6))
 (segment (start 141.086 102.046) (end 141.086 92.619) (width 0.8) (layer "B.Cu") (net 6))
 (segment (start 154.485 60.445) (end 145.985 60.445) (width 0.8) (layer "B.Cu") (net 6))
 (segment (start 143.275 90.03) (end 143.675 90.03) (width 0.8) (layer "B.Cu") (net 6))
 (segment (start 141.086 92.619) (end 143.675 90.03) (width 0.8) (layer "B.Cu") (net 6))
 (segment (start 139.72 59.017919) (end 139.72 60.22) (width 0.8) (layer "B.Cu") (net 6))
 (segment (start 143.985 58.643) (end 143.911 58.569) (width 0.8) (layer "B.Cu") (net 6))
 (segment (start 143.985 58.643) (end 144.183 58.643) (width 0.8) (layer "B.Cu") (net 6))
 (segment (start 143.911 58.569) (end 140.168919 58.569) (width 0.8) (layer "B.Cu") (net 6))
 (segment (start 158.786999 84.744313) (end 157.827078 85.704234) (width 0.8) (layer "B.Cu") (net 6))
 (segment (start 139.72 62.905) (end 139.485 63.14) (width 0.8) (layer "B.Cu") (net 6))
 (segment (start 156.485 71.177374) (end 158.787 73.479374) (width 0.8) (layer "B.Cu") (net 6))
 (segment (start 142.485 103.445) (end 141.086 102.046) (width 0.8) (layer "B.Cu") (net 6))
 (segment (start 139.72 60.22) (end 139.72 62.905) (width 0.8) (layer "B.Cu") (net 6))
 (segment (start 142.26 60.22) (end 144.709235 62.669235) (width 0.8) (layer "B.Cu") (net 3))
 (segment (start 140.727922 77.962922) (end 142.772843 75.918001) (width 0.8) (layer "B.Cu") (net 3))
 (segment (start 142.26 60.22) (end 142.26 62.915) (width 0.8) (layer "B.Cu") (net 3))
 (segment (start 154.485 79.22) (end 151.295 82.41) (width 0.8) (layer "B.Cu") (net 3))
 (segment (start 144.709235 73.981609) (end 140.727922 77.962922) (width 0.8) (layer "B.Cu") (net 3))
 (segment (start 144.709235 62.669235) (end 144.709235 73.981609) (width 0.8) (layer "B.Cu") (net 3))
 (segment (start 150.964 82.079) (end 151.295 82.41) (width 0.8) (layer "B.Cu") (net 3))
 (segment (start 142.772843 75.918001) (end 152.027157 75.918001) (width 0.8) (layer "B.Cu") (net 3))
 (segment (start 142.26 62.915) (end 142.485 63.14) (width 0.8) (layer "B.Cu") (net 3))
 (segment (start 152.027157 75.918001) (end 154.485 78.375844) (width 0.8) (layer "B.Cu") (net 3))
 (segment (start 136.683001 85.616471) (end 136.683001 82.007843) (width 0.8) (layer "B.Cu") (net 3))
 (segment (start 139.20653 88.14) (end 136.683001 85.616471) (width 0.8) (layer "B.Cu") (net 3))
 (segment (start 136.683001 82.007843) (end 140.727922 77.962922) (width 0.8) (layer "B.Cu") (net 3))
 (segment (start 139.485 88.14) (end 139.20653 88.14) (width 0.8) (layer "B.Cu") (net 3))
 (segment (start 154.485 78.375844) (end 154.485 79.22) (width 0.8) (layer "B.Cu") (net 3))
 (segment (start 144.875 82.41) (end 143.675 82.41) (width 0.8) (layer "B.Cu") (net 4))
 (segment (start 139.485 83.97) (end 141.045 82.41) (width 0.8) (layer "B.Cu") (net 4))
 (segment (start 141.045 82.41) (end 143.675 82.41) (width 0.8) (layer "B.Cu") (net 4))
 (segment (start 152.565 78.72) (end 147.365 78.72) (width 0.8) (layer "B.Cu") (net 4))
 (segment (start 146.485 94.22) (end 146.485 84.02) (width 0.8) (layer "B.Cu") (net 4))
 (segment (start 147.365 78.72) (end 143.675 82.41) (width 0.8) (layer "B.Cu") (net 4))
 (segment (start 146.485 84.02) (end 144.875 82.41) (width 0.8) (layer "B.Cu") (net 4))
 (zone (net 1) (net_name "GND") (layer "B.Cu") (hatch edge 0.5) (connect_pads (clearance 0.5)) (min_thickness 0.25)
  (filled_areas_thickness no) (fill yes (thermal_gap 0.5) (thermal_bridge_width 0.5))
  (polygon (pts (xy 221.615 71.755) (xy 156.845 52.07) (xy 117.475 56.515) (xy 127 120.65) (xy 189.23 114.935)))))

